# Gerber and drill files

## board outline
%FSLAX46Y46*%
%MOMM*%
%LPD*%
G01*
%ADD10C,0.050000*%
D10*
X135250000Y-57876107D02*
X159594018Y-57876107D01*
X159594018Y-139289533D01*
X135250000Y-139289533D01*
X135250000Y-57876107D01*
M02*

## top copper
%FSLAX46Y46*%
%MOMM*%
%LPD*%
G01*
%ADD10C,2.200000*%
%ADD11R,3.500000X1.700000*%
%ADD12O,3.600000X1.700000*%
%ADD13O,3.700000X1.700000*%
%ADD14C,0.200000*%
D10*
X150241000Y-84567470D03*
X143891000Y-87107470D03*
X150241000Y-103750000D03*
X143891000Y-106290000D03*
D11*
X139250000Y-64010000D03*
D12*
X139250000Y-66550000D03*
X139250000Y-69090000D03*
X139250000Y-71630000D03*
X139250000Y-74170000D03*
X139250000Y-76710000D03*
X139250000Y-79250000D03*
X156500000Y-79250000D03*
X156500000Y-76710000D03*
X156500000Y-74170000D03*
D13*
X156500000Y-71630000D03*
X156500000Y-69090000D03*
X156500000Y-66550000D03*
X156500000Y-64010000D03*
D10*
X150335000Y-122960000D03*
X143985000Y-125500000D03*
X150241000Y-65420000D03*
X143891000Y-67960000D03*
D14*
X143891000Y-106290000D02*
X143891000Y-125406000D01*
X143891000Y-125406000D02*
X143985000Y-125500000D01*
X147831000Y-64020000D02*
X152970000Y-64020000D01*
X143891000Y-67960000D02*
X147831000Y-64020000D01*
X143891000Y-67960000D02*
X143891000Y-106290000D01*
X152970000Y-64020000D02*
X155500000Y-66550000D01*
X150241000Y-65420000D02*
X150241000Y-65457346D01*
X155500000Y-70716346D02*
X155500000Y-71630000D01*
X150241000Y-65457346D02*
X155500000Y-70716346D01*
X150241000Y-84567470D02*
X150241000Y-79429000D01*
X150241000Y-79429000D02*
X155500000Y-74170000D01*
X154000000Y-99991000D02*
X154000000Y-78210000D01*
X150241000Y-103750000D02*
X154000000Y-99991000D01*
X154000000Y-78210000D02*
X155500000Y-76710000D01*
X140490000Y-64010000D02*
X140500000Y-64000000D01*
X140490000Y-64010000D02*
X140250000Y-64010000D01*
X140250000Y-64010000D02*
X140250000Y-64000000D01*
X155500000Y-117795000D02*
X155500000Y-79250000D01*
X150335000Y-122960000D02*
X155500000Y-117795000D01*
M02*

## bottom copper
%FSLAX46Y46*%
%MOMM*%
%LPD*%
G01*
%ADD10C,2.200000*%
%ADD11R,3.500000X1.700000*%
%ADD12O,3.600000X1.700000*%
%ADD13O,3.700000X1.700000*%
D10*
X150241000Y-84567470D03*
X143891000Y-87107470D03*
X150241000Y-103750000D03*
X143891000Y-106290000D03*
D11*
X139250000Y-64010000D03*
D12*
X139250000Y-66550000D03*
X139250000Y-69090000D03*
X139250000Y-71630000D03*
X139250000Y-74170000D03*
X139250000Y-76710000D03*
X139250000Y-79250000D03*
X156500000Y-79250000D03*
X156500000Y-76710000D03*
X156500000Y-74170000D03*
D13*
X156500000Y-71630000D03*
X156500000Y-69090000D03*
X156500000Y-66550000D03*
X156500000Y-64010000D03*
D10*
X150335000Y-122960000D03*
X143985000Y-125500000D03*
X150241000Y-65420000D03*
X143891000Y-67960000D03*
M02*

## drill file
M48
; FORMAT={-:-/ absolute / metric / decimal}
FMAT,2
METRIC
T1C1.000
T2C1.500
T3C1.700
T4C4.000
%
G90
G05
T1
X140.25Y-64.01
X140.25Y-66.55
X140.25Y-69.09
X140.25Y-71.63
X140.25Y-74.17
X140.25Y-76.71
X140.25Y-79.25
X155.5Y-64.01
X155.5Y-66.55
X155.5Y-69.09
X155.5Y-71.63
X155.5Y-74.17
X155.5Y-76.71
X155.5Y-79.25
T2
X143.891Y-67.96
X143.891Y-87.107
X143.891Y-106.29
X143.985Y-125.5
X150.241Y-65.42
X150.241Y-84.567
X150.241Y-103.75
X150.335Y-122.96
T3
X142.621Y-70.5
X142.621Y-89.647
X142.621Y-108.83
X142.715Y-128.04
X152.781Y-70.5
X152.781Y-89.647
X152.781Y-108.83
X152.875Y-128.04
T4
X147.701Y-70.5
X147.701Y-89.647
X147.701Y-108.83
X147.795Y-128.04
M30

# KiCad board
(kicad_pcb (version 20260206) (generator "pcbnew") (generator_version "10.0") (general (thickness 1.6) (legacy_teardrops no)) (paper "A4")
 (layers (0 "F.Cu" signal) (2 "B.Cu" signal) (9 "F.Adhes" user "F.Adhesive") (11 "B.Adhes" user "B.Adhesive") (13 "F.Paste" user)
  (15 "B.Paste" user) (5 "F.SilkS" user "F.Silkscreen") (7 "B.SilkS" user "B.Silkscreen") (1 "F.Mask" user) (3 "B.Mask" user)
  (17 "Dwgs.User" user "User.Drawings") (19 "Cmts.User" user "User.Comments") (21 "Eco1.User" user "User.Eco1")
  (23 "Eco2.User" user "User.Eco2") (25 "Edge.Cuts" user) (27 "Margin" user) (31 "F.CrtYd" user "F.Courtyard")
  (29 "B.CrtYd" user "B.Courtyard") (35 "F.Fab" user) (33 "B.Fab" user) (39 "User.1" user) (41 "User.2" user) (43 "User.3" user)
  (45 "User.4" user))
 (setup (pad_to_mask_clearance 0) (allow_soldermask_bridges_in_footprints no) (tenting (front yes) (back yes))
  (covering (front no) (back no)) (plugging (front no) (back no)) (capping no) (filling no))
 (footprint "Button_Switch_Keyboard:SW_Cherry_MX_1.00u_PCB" (layer "F.Cu") (at 150.241 84.56747)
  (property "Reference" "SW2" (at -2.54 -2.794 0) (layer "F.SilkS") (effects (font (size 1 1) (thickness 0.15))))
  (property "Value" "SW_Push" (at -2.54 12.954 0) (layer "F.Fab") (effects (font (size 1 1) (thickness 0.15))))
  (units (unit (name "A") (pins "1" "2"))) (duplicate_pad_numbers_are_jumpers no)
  (pad "" np_thru_hole circle (at -7.62 5.08) (size 1.7 1.7) (drill 1.7) (layers "*.Cu" "*.Mask"))
  (pad "" np_thru_hole circle (at -2.54 5.08) (size 4 4) (drill 4) (layers "*.Cu" "*.Mask"))
  (pad "" np_thru_hole circle (at 2.54 5.08) (size 1.7 1.7) (drill 1.7) (layers "*.Cu" "*.Mask"))
  (pad "1" thru_hole circle (at 0 0) (size 2.2 2.2) (drill 1.5) (layers "*.Cu" "*.Mask") (remove_unused_layers no)
   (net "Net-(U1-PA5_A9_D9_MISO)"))
  (pad "2" thru_hole circle (at -6.35 2.54) (size 2.2 2.2) (drill 1.5) (layers "*.Cu" "*.Mask") (remove_unused_layers no) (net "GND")))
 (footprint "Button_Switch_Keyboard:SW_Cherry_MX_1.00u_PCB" (layer "F.Cu") (at 150.241 103.75)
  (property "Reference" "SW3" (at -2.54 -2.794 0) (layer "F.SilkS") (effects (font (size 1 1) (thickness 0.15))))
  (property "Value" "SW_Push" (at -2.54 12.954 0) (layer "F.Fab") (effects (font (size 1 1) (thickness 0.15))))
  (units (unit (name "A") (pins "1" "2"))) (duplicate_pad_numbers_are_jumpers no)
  (pad "" np_thru_hole circle (at -7.62 5.08) (size 1.7 1.7) (drill 1.7) (layers "*.Cu" "*.Mask"))
  (pad "" np_thru_hole circle (at -2.54 5.08) (size 4 4) (drill 4) (layers "*.Cu" "*.Mask"))
  (pad "" np_thru_hole circle (at 2.54 5.08) (size 1.7 1.7) (drill 1.7) (layers "*.Cu" "*.Mask"))
  (pad "1" thru_hole circle (at 0 0) (size 2.2 2.2) (drill 1.5) (layers "*.Cu" "*.Mask") (remove_unused_layers no)
   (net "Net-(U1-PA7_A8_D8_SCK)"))
  (pad "2" thru_hole circle (at -6.35 2.54) (size 2.2 2.2) (drill 1.5) (layers "*.Cu" "*.Mask") (remove_unused_layers no) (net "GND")))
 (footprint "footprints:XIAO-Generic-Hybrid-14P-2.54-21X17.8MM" (layer "F.Cu") (at 147.875 71.63)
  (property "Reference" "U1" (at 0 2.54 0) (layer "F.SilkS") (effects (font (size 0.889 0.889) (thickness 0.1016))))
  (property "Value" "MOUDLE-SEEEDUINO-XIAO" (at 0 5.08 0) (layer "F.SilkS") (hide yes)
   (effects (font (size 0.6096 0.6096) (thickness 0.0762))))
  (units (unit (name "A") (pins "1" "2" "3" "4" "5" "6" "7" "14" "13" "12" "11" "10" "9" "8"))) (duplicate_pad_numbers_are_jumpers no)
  (pad "1" thru_hole rect (at -7.625 -7.62) (size 3.5 1.7) (drill 1 (offset -1 0)) (layers "*.Cu" "*.Mask") (remove_unused_layers no)
   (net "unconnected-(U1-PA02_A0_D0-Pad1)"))
  (pad "2" thru_hole oval (at -7.625 -5.08) (size 3.6 1.7) (drill 1 (offset -1 0)) (layers "*.Cu" "*.Mask") (remove_unused_layers no)
   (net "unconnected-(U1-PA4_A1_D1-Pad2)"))
  (pad "3" thru_hole oval (at -7.625 -2.54) (size 3.6 1.7) (drill 1 (offset -1 0)) (layers "*.Cu" "*.Mask") (remove_unused_layers no)
   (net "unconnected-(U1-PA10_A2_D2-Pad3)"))
  (pad "4" thru_hole oval (at -7.625 0) (size 3.6 1.7) (drill 1 (offset -1 0)) (layers "*.Cu" "*.Mask") (remove_unused_layers no)
   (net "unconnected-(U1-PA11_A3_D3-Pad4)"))
  (pad "5" thru_hole oval (at -7.625 2.54) (size 3.6 1.7) (drill 1 (offset -1 0)) (layers "*.Cu" "*.Mask") (remove_unused_layers no)
   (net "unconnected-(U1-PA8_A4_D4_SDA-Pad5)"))
  (pad "6" thru_hole oval (at -7.625 5.08 180) (size 3.6 1.7) (drill 1 (offset 1 0)) (layers "*.Cu" "*.Mask") (remove_unused_layers no)
   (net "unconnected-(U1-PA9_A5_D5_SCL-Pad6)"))
  (pad "7" thru_hole oval (at -7.625 7.62) (size 3.6 1.7) (drill 1 (offset -1 0)) (layers "*.Cu" "*.Mask") (remove_unused_layers no)
   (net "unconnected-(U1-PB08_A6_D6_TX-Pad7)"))
  (pad "8" thru_hole oval (at 7.625 7.62) (size 3.6 1.7) (drill 1 (offset 1 0)) (layers "*.Cu" "*.Mask") (remove_unused_layers no)
   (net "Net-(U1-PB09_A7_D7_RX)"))
  (pad "9" thru_hole oval (at 7.625 5.08) (size 3.6 1.7) (drill 1 (offset 1 0)) (layers "*.Cu" "*.Mask") (remove_unused_layers no)
   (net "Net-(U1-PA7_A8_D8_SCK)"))
  (pad "10" thru_hole oval (at 7.625 2.54) (size 3.6 1.7) (drill 1 (offset 1 0)) (layers "*.Cu" "*.Mask") (remove_unused_layers no)
   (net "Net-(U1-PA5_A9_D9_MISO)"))
  (pad "11" thru_hole oval (at 7.625 0) (size 3.7 1.7) (drill 1 (offset 1 0)) (layers "*.Cu" "*.Mask") (remove_unused_layers no)
   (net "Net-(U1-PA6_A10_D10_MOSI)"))
  (pad "12" thru_hole oval (at 7.625 -2.54) (size 3.7 1.7) (drill 1 (offset 1 0)) (layers "*.Cu" "*.Mask") (remove_unused_layers no)
   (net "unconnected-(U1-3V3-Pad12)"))
  (pad "13" thru_hole oval (at 7.625 -5.08) (size 3.7 1.7) (drill 1 (offset 1 0)) (layers "*.Cu" "*.Mask") (remove_unused_layers no)
   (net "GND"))
  (pad "14" thru_hole oval (at 7.625 -7.62) (size 3.7 1.7) (drill 1 (offset 1 0)) (layers "*.Cu" "*.Mask") (remove_unused_layers no)
   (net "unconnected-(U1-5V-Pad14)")))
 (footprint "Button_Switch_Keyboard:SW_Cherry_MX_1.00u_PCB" (layer "F.Cu") (at 150.335 122.96)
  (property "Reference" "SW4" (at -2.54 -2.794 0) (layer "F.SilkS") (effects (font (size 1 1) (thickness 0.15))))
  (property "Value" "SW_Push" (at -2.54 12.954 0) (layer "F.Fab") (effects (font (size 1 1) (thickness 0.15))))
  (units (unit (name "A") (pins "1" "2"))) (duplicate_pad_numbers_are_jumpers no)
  (pad "" np_thru_hole circle (at -7.62 5.08) (size 1.7 1.7) (drill 1.7) (layers "*.Cu" "*.Mask"))
  (pad "" np_thru_hole circle (at -2.54 5.08) (size 4 4) (drill 4) (layers "*.Cu" "*.Mask"))
  (pad "" np_thru_hole circle (at 2.54 5.08) (size 1.7 1.7) (drill 1.7) (layers "*.Cu" "*.Mask"))
  (pad "1" thru_hole circle (at 0 0) (size 2.2 2.2) (drill 1.5) (layers "*.Cu" "*.Mask") (remove_unused_layers no)
   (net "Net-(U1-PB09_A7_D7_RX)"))
  (pad "2" thru_hole circle (at -6.35 2.54) (size 2.2 2.2) (drill 1.5) (layers "*.Cu" "*.Mask") (remove_unused_layers no) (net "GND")))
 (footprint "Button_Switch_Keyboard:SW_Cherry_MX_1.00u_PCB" (layer "F.Cu") (at 150.241 65.42)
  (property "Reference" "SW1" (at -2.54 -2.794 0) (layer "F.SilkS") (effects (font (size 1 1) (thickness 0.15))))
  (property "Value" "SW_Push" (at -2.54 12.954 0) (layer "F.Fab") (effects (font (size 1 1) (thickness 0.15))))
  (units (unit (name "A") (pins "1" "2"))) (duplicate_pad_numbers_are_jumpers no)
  (pad "" np_thru_hole circle (at -7.62 5.08) (size 1.7 1.7) (drill 1.7) (layers "*.Cu" "*.Mask"))
  (pad "" np_thru_hole circle (at -2.54 5.08) (size 4 4) (drill 4) (layers "*.Cu" "*.Mask"))
  (pad "" np_thru_hole circle (at 2.54 5.08) (size 1.7 1.7) (drill 1.7) (layers "*.Cu" "*.Mask"))
  (pad "1" thru_hole circle (at 0 0) (size 2.2 2.2) (drill 1.5) (layers "*.Cu" "*.Mask") (remove_unused_layers no)
   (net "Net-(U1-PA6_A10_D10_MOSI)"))
  (pad "2" thru_hole circle (at -6.35 2.54) (size 2.2 2.2) (drill 1.5) (layers "*.Cu" "*.Mask") (remove_unused_layers no) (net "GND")))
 (gr_rect (start 135.25 57.876107) (end 159.594018 139.289533) (stroke (width 0.05) (type default)) (fill no) (layer "Edge.Cuts"))
 (segment (start 143.891 106.29) (end 143.891 125.406) (width 0.2) (layer "F.Cu") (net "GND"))
 (segment (start 143.891 125.406) (end 143.985 125.5) (width 0.2) (layer "F.Cu") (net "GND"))
 (segment (start 147.831 64.02) (end 152.97 64.02) (width 0.2) (layer "F.Cu") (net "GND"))
 (segment (start 143.891 67.96) (end 147.831 64.02) (width 0.2) (layer "F.Cu") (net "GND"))
 (segment (start 143.891 67.96) (end 143.891 106.29) (width 0.2) (layer "F.Cu") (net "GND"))
 (segment (start 152.97 64.02) (end 155.5 66.55) (width 0.2) (layer "F.Cu") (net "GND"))
 (segment (start 150.241 65.42) (end 150.241 65.457346) (width 0.2) (layer "F.Cu") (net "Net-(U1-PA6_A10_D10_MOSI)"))
 (segment (start 155.5 70.716346) (end 155.5 71.63) (width 0.2) (layer "F.Cu") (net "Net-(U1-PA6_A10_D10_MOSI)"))
 (segment (start 150.241 65.457346) (end 155.5 70.716346) (width 0.2) (layer "F.Cu") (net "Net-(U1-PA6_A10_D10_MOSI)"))
 (segment (start 150.241 84.56747) (end 150.241 79.429) (width 0.2) (layer "F.Cu") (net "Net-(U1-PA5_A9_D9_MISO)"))
 (segment (start 150.241 79.429) (end 155.5 74.17) (width 0.2) (layer "F.Cu") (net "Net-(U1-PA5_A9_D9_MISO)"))
 (segment (start 154 99.991) (end 154 78.21) (width 0.2) (layer "F.Cu") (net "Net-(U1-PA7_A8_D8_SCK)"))
 (segment (start 150.241 103.75) (end 154 99.991) (width 0.2) (layer "F.Cu") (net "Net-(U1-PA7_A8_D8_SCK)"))
 (segment (start 154 78.21) (end 155.5 76.71) (width 0.2) (layer "F.Cu") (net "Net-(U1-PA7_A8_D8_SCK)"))
 (segment (start 140.49 64.01) (end 140.5 64) (width 0.2) (layer "F.Cu") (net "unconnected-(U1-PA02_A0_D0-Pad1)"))
 (segment (start 140.49 64.01) (end 140.25 64.01) (width 0.2) (layer "F.Cu") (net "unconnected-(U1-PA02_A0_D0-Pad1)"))
 (segment (start 140.25 64.01) (end 140.25 64) (width 0.2) (layer "F.Cu") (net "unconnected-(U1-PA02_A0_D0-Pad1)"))
 (segment (start 155.5 117.795) (end 155.5 79.25) (width 0.2) (layer "F.Cu") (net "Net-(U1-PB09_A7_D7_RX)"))
 (segment (start 150.335 122.96) (end 155.5 117.795) (width 0.2) (layer "F.Cu") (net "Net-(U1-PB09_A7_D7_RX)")))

